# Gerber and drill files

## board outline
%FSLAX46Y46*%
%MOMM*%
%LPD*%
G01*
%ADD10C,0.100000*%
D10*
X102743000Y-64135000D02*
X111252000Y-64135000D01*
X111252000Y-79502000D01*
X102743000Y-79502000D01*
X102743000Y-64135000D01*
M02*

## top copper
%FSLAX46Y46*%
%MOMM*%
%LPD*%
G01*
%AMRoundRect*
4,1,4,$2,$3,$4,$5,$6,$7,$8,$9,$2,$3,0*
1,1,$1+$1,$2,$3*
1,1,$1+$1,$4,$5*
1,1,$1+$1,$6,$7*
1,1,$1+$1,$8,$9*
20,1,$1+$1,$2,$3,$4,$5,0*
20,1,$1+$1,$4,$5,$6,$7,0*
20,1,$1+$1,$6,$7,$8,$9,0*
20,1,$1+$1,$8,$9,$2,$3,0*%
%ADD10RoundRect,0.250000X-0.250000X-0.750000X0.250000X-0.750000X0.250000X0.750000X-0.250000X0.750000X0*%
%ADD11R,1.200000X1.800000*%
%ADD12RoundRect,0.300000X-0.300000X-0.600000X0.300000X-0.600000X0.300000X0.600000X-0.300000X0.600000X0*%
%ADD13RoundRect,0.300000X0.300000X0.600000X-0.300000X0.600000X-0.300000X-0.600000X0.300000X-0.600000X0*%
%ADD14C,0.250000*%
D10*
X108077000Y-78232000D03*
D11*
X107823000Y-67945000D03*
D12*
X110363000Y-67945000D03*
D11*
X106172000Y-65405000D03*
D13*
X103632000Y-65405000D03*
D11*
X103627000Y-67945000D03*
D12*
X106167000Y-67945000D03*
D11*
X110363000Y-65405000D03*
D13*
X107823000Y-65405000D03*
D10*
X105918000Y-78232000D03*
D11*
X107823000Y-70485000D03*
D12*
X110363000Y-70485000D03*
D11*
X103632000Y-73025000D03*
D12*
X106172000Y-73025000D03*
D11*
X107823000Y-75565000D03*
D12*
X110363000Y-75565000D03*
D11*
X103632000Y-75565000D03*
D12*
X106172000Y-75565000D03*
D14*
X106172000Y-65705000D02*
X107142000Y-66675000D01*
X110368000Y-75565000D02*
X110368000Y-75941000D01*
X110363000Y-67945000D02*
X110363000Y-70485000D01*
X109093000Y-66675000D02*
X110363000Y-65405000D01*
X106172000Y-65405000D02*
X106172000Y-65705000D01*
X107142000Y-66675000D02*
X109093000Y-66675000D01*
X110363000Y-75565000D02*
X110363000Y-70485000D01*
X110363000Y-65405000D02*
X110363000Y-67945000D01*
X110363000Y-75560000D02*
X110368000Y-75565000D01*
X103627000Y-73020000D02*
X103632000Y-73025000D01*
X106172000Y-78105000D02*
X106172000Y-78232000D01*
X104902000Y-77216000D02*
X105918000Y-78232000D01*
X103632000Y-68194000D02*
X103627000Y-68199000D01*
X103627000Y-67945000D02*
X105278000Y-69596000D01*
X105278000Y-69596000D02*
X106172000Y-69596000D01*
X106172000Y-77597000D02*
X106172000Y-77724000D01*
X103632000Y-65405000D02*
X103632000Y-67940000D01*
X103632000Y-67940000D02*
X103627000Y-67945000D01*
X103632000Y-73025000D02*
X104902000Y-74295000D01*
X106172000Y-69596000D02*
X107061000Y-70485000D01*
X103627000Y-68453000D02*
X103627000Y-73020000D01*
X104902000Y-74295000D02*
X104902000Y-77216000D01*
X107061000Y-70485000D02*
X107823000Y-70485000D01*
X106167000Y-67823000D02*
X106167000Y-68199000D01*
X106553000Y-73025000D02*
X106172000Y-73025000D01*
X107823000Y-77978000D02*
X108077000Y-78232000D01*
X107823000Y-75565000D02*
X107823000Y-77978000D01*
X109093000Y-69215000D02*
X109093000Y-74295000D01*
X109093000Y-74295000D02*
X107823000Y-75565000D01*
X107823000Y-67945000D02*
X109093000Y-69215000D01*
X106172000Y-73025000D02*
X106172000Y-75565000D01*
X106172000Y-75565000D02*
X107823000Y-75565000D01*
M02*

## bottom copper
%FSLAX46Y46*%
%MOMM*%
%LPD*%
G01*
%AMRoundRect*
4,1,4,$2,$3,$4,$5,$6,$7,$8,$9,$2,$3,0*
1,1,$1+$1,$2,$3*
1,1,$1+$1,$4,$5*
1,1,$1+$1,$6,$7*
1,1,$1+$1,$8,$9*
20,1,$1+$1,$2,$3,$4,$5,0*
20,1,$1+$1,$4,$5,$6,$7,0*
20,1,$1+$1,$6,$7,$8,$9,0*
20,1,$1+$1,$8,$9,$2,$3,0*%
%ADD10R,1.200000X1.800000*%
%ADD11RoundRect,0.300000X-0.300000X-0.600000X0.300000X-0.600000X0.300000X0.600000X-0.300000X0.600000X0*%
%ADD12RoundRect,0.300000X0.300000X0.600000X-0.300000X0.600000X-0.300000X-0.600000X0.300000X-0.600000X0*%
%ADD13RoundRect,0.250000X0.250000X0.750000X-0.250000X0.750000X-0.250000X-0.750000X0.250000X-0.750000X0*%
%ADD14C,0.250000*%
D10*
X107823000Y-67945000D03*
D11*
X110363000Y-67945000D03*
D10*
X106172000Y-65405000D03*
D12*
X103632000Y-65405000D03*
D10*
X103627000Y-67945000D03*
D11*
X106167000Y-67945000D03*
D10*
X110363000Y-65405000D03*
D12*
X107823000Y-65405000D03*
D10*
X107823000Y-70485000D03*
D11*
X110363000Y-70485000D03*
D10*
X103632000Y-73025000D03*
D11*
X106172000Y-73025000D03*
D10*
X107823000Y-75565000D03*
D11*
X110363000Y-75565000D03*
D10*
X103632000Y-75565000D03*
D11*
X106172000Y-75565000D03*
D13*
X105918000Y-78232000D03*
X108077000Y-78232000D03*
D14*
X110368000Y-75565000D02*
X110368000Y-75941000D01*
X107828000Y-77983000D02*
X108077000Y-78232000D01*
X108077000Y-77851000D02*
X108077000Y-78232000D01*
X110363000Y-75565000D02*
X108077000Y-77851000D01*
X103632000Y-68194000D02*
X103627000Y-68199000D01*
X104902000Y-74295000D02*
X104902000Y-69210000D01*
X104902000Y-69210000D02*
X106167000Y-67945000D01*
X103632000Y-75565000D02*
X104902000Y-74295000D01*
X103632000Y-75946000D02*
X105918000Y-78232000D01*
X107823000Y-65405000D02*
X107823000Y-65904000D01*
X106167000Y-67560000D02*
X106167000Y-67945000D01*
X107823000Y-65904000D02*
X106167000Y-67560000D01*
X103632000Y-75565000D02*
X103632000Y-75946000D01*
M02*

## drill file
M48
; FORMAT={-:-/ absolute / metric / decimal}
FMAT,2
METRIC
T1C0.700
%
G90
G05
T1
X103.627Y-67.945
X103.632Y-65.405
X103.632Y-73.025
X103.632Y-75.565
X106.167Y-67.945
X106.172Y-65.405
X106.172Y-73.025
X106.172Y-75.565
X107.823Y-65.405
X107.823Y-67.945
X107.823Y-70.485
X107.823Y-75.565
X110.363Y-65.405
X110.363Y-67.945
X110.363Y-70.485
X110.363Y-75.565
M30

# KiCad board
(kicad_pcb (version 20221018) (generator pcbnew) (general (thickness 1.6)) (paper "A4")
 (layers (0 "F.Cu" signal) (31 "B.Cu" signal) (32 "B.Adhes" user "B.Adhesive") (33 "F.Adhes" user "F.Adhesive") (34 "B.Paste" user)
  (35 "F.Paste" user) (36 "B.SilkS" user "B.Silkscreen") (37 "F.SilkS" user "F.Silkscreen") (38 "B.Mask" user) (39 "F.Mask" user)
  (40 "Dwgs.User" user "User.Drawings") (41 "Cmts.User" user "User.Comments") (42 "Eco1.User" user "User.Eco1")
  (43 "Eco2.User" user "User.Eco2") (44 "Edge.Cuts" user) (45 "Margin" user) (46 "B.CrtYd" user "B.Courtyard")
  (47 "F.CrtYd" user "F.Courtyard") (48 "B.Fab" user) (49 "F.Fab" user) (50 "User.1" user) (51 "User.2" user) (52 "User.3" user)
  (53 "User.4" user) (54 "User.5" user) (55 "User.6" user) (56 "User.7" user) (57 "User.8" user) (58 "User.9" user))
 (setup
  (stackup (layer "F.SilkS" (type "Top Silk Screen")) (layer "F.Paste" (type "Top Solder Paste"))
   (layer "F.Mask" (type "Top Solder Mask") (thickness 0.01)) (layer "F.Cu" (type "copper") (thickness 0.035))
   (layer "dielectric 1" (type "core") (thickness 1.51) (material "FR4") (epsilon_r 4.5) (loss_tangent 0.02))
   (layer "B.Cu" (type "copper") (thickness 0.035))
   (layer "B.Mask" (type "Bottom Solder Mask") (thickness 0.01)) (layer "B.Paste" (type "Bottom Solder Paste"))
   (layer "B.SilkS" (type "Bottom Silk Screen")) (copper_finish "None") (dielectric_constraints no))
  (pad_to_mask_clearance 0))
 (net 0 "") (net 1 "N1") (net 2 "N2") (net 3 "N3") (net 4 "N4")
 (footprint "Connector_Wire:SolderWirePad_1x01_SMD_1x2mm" (layer "F.Cu") (at 108.077 78.232)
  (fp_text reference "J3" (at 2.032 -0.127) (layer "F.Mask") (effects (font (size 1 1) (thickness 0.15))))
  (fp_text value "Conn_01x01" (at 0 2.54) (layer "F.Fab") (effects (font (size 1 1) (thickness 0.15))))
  (pad "1" smd roundrect (at 0 0) (size 1 2) (layers "F.Cu" "F.Paste" "F.Mask") (roundrect_rratio 0.25) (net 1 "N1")))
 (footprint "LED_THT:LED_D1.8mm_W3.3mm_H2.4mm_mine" (layer "F.Cu") (at 107.823 67.945)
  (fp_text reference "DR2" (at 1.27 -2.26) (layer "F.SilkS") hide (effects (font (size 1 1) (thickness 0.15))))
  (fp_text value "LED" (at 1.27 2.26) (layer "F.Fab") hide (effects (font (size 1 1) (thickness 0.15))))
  (pad "1" thru_hole rect (at 0 0) (size 1.2 1.8) (drill 0.7) (layers "*.Cu" "*.Mask") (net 1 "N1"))
  (pad "2" thru_hole roundrect (at 2.54 0) (size 1.2 1.8) (drill 0.7) (layers "*.Cu" "*.Mask") (roundrect_rratio 0.25) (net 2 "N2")))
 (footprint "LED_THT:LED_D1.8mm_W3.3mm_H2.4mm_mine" (layer "F.Cu") (at 106.172 65.405 180)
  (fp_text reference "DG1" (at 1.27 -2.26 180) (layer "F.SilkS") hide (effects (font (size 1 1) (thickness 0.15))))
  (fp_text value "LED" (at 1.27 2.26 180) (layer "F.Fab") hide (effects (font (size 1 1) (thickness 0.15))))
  (pad "1" thru_hole rect (at 0 0 180) (size 1.2 1.8) (drill 0.7) (layers "*.Cu" "*.Mask") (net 2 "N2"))
  (pad "2" thru_hole roundrect (at 2.54 0 180) (size 1.2 1.8) (drill 0.7) (layers "*.Cu" "*.Mask") (roundrect_rratio 0.25) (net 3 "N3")))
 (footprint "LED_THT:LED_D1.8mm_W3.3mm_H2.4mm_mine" (layer "F.Cu") (at 103.627 67.945)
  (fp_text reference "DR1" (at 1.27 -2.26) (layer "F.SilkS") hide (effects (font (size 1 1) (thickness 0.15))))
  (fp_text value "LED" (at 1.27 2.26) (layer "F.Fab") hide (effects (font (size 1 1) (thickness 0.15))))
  (pad "1" thru_hole rect (at 0 0) (size 1.2 1.8) (drill 0.7) (layers "*.Cu" "*.Mask") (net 3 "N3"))
  (pad "2" thru_hole roundrect (at 2.54 0) (size 1.2 1.8) (drill 0.7) (layers "*.Cu" "*.Mask") (roundrect_rratio 0.25) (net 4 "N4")))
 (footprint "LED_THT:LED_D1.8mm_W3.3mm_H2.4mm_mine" (layer "F.Cu") (at 110.363 65.405 180)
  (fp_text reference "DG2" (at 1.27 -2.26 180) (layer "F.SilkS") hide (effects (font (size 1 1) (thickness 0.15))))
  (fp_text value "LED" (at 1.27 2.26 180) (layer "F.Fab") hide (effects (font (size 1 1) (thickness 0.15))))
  (pad "1" thru_hole rect (at 0 0 180) (size 1.2 1.8) (drill 0.7) (layers "*.Cu" "*.Mask") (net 2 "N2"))
  (pad "2" thru_hole roundrect (at 2.54 0 180) (size 1.2 1.8) (drill 0.7) (layers "*.Cu" "*.Mask") (roundrect_rratio 0.25) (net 4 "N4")))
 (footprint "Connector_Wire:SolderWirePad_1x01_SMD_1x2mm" (layer "F.Cu") (at 105.918 78.232)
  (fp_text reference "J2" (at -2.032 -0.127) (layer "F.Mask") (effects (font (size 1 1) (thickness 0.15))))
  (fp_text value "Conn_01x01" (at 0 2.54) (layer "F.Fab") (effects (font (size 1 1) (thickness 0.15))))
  (pad "1" smd roundrect (at 0 0) (size 1 2) (layers "F.Cu" "F.Paste" "F.Mask") (roundrect_rratio 0.25) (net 3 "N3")))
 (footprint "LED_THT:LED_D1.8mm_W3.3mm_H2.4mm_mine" (layer "F.Cu") (at 107.823 70.485)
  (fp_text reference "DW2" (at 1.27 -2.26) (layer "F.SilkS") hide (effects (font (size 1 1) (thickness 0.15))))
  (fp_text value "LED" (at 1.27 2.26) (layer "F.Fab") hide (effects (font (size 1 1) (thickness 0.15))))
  (pad "1" thru_hole rect (at 0 0) (size 1.2 1.8) (drill 0.7) (layers "*.Cu" "*.Mask") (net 3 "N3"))
  (pad "2" thru_hole roundrect (at 2.54 0) (size 1.2 1.8) (drill 0.7) (layers "*.Cu" "*.Mask") (roundrect_rratio 0.25) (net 2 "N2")))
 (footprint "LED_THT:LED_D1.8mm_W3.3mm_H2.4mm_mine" (layer "F.Cu") (at 103.632 73.025)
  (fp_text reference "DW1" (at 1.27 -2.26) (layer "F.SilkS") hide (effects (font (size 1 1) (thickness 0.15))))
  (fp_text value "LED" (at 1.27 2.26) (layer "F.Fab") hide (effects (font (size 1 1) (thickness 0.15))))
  (pad "1" thru_hole rect (at 0 0) (size 1.2 1.8) (drill 0.7) (layers "*.Cu" "*.Mask") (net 3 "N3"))
  (pad "2" thru_hole roundrect (at 2.54 0) (size 1.2 1.8) (drill 0.7) (layers "*.Cu" "*.Mask") (roundrect_rratio 0.25) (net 1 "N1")))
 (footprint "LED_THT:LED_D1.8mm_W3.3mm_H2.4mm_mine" (layer "B.Cu") (at 107.823 75.565)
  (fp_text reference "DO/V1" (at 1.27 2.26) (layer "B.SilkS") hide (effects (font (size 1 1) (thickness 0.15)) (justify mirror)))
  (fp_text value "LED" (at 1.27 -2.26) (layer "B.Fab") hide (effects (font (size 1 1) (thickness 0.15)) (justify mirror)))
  (pad "1" thru_hole rect (at 0 0) (size 1.2 1.8) (drill 0.7) (layers "*.Cu" "*.Mask") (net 1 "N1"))
  (pad "2" thru_hole roundrect (at 2.54 0) (size 1.2 1.8) (drill 0.7) (layers "*.Cu" "*.Mask") (roundrect_rratio 0.25) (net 2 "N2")))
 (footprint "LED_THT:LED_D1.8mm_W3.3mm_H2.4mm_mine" (layer "B.Cu") (at 103.632 75.565)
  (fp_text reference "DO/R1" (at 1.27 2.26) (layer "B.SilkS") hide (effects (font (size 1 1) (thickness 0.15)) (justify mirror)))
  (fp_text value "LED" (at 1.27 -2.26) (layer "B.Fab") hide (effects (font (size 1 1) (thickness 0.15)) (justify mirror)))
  (pad "1" thru_hole rect (at 0 0) (size 1.2 1.8) (drill 0.7) (layers "*.Cu" "*.Mask") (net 4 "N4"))
  (pad "2" thru_hole roundrect (at 2.54 0) (size 1.2 1.8) (drill 0.7) (layers "*.Cu" "*.Mask") (roundrect_rratio 0.25) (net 1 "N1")))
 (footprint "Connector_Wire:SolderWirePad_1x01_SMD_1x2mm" (layer "B.Cu") (at 105.918 78.232 180)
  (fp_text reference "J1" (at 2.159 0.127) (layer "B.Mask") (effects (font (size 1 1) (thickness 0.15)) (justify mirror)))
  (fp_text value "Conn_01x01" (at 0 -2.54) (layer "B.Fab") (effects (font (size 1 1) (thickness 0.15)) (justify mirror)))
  (pad "1" smd roundrect (at 0 0 180) (size 1 2) (layers "B.Cu" "B.Paste" "B.Mask") (roundrect_rratio 0.25) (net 4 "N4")))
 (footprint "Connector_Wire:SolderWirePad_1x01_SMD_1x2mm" (layer "B.Cu") (at 108.077 78.232 180)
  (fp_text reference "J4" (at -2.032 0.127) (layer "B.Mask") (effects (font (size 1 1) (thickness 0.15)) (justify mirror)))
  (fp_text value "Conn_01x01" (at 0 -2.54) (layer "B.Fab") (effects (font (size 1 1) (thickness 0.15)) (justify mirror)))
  (pad "1" smd roundrect (at 0 0 180) (size 1 2) (layers "B.Cu" "B.Paste" "B.Mask") (roundrect_rratio 0.25) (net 2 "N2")))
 (gr_rect (start 102.743 64.135) (end 111.252 79.502) (stroke (width 0.1) (type default)) (fill none) (layer "Edge.Cuts"))
 (segment (start 106.172 65.705) (end 107.142 66.675) (width 0.25) (layer "F.Cu") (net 2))
 (segment (start 110.368 75.565) (end 110.368 75.941) (width 0.25) (layer "F.Cu") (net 2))
 (segment (start 110.363 67.945) (end 110.363 70.485) (width 0.25) (layer "F.Cu") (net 2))
 (segment (start 109.093 66.675) (end 110.363 65.405) (width 0.25) (layer "F.Cu") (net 2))
 (segment (start 106.172 65.405) (end 106.172 65.705) (width 0.25) (layer "F.Cu") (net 2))
 (segment (start 107.142 66.675) (end 109.093 66.675) (width 0.25) (layer "F.Cu") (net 2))
 (segment (start 110.363 75.565) (end 110.363 70.485) (width 0.25) (layer "F.Cu") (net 2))
 (segment (start 110.363 65.405) (end 110.363 67.945) (width 0.25) (layer "F.Cu") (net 2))
 (segment (start 110.363 75.56) (end 110.368 75.565) (width 0.25) (layer "F.Cu") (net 2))
 (segment (start 110.368 75.565) (end 110.368 75.941) (width 0.25) (layer "B.Cu") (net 2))
 (segment (start 107.828 77.983) (end 108.077 78.232) (width 0.25) (layer "B.Cu") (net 2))
 (segment (start 108.077 77.851) (end 108.077 78.232) (width 0.25) (layer "B.Cu") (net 2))
 (segment (start 110.363 75.565) (end 108.077 77.851) (width 0.25) (layer "B.Cu") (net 2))
 (segment (start 103.627 73.02) (end 103.632 73.025) (width 0.25) (layer "F.Cu") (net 3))
 (segment (start 106.172 78.105) (end 106.172 78.232) (width 0.25) (layer "F.Cu") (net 3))
 (segment (start 104.902 77.216) (end 105.918 78.232) (width 0.25) (layer "F.Cu") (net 3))
 (segment (start 103.632 68.194) (end 103.627 68.199) (width 0.25) (layer "F.Cu") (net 3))
 (segment (start 103.627 67.945) (end 105.278 69.596) (width 0.25) (layer "F.Cu") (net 3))
 (segment (start 105.278 69.596) (end 106.172 69.596) (width 0.25) (layer "F.Cu") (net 3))
 (segment (start 106.172 77.597) (end 106.172 77.724) (width 0.25) (layer "F.Cu") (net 3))
 (segment (start 103.632 65.405) (end 103.632 67.94) (width 0.25) (layer "F.Cu") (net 3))
 (segment (start 103.632 67.94) (end 103.627 67.945) (width 0.25) (layer "F.Cu") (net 3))
 (segment (start 103.632 73.025) (end 104.902 74.295) (width 0.25) (layer "F.Cu") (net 3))
 (segment (start 106.172 69.596) (end 107.061 70.485) (width 0.25) (layer "F.Cu") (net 3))
 (segment (start 103.627 68.453) (end 103.627 73.02) (width 0.25) (layer "F.Cu") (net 3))
 (segment (start 104.902 74.295) (end 104.902 77.216) (width 0.25) (layer "F.Cu") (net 3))
 (segment (start 107.061 70.485) (end 107.823 70.485) (width 0.25) (layer "F.Cu") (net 3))
 (segment (start 103.632 68.194) (end 103.627 68.199) (width 0.25) (layer "B.Cu") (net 3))
 (segment (start 106.167 67.823) (end 106.167 68.199) (width 0.25) (layer "F.Cu") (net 4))
 (segment (start 104.902 74.295) (end 104.902 69.21) (width 0.25) (layer "B.Cu") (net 4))
 (segment (start 104.902 69.21) (end 106.167 67.945) (width 0.25) (layer "B.Cu") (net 4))
 (segment (start 103.632 75.565) (end 104.902 74.295) (width 0.25) (layer "B.Cu") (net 4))
 (segment (start 103.632 75.946) (end 105.918 78.232) (width 0.25) (layer "B.Cu") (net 4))
 (segment (start 107.823 65.405) (end 107.823 65.904) (width 0.25) (layer "B.Cu") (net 4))
 (segment (start 106.167 67.56) (end 106.167 67.945) (width 0.25) (layer "B.Cu") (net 4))
 (segment (start 107.823 65.904) (end 106.167 67.56) (width 0.25) (layer "B.Cu") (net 4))
 (segment (start 103.632 75.565) (end 103.632 75.946) (width 0.25) (layer "B.Cu") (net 4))
 (segment (start 106.553 73.025) (end 106.172 73.025) (width 0.25) (layer "F.Cu") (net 1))
 (segment (start 107.823 77.978) (end 108.077 78.232) (width 0.25) (layer "F.Cu") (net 1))
 (segment (start 107.823 75.565) (end 107.823 77.978) (width 0.25) (layer "F.Cu") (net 1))
 (segment (start 109.093 69.215) (end 109.093 74.295) (width 0.25) (layer "F.Cu") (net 1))
 (segment (start 109.093 74.295) (end 107.823 75.565) (width 0.25) (layer "F.Cu") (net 1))
 (segment (start 107.823 67.945) (end 109.093 69.215) (width 0.25) (layer "F.Cu") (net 1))
 (segment (start 106.172 73.025) (end 106.172 75.565) (width 0.25) (layer "F.Cu") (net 1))
 (segment (start 106.172 75.565) (end 107.823 75.565) (width 0.25) (layer "F.Cu") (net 1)))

